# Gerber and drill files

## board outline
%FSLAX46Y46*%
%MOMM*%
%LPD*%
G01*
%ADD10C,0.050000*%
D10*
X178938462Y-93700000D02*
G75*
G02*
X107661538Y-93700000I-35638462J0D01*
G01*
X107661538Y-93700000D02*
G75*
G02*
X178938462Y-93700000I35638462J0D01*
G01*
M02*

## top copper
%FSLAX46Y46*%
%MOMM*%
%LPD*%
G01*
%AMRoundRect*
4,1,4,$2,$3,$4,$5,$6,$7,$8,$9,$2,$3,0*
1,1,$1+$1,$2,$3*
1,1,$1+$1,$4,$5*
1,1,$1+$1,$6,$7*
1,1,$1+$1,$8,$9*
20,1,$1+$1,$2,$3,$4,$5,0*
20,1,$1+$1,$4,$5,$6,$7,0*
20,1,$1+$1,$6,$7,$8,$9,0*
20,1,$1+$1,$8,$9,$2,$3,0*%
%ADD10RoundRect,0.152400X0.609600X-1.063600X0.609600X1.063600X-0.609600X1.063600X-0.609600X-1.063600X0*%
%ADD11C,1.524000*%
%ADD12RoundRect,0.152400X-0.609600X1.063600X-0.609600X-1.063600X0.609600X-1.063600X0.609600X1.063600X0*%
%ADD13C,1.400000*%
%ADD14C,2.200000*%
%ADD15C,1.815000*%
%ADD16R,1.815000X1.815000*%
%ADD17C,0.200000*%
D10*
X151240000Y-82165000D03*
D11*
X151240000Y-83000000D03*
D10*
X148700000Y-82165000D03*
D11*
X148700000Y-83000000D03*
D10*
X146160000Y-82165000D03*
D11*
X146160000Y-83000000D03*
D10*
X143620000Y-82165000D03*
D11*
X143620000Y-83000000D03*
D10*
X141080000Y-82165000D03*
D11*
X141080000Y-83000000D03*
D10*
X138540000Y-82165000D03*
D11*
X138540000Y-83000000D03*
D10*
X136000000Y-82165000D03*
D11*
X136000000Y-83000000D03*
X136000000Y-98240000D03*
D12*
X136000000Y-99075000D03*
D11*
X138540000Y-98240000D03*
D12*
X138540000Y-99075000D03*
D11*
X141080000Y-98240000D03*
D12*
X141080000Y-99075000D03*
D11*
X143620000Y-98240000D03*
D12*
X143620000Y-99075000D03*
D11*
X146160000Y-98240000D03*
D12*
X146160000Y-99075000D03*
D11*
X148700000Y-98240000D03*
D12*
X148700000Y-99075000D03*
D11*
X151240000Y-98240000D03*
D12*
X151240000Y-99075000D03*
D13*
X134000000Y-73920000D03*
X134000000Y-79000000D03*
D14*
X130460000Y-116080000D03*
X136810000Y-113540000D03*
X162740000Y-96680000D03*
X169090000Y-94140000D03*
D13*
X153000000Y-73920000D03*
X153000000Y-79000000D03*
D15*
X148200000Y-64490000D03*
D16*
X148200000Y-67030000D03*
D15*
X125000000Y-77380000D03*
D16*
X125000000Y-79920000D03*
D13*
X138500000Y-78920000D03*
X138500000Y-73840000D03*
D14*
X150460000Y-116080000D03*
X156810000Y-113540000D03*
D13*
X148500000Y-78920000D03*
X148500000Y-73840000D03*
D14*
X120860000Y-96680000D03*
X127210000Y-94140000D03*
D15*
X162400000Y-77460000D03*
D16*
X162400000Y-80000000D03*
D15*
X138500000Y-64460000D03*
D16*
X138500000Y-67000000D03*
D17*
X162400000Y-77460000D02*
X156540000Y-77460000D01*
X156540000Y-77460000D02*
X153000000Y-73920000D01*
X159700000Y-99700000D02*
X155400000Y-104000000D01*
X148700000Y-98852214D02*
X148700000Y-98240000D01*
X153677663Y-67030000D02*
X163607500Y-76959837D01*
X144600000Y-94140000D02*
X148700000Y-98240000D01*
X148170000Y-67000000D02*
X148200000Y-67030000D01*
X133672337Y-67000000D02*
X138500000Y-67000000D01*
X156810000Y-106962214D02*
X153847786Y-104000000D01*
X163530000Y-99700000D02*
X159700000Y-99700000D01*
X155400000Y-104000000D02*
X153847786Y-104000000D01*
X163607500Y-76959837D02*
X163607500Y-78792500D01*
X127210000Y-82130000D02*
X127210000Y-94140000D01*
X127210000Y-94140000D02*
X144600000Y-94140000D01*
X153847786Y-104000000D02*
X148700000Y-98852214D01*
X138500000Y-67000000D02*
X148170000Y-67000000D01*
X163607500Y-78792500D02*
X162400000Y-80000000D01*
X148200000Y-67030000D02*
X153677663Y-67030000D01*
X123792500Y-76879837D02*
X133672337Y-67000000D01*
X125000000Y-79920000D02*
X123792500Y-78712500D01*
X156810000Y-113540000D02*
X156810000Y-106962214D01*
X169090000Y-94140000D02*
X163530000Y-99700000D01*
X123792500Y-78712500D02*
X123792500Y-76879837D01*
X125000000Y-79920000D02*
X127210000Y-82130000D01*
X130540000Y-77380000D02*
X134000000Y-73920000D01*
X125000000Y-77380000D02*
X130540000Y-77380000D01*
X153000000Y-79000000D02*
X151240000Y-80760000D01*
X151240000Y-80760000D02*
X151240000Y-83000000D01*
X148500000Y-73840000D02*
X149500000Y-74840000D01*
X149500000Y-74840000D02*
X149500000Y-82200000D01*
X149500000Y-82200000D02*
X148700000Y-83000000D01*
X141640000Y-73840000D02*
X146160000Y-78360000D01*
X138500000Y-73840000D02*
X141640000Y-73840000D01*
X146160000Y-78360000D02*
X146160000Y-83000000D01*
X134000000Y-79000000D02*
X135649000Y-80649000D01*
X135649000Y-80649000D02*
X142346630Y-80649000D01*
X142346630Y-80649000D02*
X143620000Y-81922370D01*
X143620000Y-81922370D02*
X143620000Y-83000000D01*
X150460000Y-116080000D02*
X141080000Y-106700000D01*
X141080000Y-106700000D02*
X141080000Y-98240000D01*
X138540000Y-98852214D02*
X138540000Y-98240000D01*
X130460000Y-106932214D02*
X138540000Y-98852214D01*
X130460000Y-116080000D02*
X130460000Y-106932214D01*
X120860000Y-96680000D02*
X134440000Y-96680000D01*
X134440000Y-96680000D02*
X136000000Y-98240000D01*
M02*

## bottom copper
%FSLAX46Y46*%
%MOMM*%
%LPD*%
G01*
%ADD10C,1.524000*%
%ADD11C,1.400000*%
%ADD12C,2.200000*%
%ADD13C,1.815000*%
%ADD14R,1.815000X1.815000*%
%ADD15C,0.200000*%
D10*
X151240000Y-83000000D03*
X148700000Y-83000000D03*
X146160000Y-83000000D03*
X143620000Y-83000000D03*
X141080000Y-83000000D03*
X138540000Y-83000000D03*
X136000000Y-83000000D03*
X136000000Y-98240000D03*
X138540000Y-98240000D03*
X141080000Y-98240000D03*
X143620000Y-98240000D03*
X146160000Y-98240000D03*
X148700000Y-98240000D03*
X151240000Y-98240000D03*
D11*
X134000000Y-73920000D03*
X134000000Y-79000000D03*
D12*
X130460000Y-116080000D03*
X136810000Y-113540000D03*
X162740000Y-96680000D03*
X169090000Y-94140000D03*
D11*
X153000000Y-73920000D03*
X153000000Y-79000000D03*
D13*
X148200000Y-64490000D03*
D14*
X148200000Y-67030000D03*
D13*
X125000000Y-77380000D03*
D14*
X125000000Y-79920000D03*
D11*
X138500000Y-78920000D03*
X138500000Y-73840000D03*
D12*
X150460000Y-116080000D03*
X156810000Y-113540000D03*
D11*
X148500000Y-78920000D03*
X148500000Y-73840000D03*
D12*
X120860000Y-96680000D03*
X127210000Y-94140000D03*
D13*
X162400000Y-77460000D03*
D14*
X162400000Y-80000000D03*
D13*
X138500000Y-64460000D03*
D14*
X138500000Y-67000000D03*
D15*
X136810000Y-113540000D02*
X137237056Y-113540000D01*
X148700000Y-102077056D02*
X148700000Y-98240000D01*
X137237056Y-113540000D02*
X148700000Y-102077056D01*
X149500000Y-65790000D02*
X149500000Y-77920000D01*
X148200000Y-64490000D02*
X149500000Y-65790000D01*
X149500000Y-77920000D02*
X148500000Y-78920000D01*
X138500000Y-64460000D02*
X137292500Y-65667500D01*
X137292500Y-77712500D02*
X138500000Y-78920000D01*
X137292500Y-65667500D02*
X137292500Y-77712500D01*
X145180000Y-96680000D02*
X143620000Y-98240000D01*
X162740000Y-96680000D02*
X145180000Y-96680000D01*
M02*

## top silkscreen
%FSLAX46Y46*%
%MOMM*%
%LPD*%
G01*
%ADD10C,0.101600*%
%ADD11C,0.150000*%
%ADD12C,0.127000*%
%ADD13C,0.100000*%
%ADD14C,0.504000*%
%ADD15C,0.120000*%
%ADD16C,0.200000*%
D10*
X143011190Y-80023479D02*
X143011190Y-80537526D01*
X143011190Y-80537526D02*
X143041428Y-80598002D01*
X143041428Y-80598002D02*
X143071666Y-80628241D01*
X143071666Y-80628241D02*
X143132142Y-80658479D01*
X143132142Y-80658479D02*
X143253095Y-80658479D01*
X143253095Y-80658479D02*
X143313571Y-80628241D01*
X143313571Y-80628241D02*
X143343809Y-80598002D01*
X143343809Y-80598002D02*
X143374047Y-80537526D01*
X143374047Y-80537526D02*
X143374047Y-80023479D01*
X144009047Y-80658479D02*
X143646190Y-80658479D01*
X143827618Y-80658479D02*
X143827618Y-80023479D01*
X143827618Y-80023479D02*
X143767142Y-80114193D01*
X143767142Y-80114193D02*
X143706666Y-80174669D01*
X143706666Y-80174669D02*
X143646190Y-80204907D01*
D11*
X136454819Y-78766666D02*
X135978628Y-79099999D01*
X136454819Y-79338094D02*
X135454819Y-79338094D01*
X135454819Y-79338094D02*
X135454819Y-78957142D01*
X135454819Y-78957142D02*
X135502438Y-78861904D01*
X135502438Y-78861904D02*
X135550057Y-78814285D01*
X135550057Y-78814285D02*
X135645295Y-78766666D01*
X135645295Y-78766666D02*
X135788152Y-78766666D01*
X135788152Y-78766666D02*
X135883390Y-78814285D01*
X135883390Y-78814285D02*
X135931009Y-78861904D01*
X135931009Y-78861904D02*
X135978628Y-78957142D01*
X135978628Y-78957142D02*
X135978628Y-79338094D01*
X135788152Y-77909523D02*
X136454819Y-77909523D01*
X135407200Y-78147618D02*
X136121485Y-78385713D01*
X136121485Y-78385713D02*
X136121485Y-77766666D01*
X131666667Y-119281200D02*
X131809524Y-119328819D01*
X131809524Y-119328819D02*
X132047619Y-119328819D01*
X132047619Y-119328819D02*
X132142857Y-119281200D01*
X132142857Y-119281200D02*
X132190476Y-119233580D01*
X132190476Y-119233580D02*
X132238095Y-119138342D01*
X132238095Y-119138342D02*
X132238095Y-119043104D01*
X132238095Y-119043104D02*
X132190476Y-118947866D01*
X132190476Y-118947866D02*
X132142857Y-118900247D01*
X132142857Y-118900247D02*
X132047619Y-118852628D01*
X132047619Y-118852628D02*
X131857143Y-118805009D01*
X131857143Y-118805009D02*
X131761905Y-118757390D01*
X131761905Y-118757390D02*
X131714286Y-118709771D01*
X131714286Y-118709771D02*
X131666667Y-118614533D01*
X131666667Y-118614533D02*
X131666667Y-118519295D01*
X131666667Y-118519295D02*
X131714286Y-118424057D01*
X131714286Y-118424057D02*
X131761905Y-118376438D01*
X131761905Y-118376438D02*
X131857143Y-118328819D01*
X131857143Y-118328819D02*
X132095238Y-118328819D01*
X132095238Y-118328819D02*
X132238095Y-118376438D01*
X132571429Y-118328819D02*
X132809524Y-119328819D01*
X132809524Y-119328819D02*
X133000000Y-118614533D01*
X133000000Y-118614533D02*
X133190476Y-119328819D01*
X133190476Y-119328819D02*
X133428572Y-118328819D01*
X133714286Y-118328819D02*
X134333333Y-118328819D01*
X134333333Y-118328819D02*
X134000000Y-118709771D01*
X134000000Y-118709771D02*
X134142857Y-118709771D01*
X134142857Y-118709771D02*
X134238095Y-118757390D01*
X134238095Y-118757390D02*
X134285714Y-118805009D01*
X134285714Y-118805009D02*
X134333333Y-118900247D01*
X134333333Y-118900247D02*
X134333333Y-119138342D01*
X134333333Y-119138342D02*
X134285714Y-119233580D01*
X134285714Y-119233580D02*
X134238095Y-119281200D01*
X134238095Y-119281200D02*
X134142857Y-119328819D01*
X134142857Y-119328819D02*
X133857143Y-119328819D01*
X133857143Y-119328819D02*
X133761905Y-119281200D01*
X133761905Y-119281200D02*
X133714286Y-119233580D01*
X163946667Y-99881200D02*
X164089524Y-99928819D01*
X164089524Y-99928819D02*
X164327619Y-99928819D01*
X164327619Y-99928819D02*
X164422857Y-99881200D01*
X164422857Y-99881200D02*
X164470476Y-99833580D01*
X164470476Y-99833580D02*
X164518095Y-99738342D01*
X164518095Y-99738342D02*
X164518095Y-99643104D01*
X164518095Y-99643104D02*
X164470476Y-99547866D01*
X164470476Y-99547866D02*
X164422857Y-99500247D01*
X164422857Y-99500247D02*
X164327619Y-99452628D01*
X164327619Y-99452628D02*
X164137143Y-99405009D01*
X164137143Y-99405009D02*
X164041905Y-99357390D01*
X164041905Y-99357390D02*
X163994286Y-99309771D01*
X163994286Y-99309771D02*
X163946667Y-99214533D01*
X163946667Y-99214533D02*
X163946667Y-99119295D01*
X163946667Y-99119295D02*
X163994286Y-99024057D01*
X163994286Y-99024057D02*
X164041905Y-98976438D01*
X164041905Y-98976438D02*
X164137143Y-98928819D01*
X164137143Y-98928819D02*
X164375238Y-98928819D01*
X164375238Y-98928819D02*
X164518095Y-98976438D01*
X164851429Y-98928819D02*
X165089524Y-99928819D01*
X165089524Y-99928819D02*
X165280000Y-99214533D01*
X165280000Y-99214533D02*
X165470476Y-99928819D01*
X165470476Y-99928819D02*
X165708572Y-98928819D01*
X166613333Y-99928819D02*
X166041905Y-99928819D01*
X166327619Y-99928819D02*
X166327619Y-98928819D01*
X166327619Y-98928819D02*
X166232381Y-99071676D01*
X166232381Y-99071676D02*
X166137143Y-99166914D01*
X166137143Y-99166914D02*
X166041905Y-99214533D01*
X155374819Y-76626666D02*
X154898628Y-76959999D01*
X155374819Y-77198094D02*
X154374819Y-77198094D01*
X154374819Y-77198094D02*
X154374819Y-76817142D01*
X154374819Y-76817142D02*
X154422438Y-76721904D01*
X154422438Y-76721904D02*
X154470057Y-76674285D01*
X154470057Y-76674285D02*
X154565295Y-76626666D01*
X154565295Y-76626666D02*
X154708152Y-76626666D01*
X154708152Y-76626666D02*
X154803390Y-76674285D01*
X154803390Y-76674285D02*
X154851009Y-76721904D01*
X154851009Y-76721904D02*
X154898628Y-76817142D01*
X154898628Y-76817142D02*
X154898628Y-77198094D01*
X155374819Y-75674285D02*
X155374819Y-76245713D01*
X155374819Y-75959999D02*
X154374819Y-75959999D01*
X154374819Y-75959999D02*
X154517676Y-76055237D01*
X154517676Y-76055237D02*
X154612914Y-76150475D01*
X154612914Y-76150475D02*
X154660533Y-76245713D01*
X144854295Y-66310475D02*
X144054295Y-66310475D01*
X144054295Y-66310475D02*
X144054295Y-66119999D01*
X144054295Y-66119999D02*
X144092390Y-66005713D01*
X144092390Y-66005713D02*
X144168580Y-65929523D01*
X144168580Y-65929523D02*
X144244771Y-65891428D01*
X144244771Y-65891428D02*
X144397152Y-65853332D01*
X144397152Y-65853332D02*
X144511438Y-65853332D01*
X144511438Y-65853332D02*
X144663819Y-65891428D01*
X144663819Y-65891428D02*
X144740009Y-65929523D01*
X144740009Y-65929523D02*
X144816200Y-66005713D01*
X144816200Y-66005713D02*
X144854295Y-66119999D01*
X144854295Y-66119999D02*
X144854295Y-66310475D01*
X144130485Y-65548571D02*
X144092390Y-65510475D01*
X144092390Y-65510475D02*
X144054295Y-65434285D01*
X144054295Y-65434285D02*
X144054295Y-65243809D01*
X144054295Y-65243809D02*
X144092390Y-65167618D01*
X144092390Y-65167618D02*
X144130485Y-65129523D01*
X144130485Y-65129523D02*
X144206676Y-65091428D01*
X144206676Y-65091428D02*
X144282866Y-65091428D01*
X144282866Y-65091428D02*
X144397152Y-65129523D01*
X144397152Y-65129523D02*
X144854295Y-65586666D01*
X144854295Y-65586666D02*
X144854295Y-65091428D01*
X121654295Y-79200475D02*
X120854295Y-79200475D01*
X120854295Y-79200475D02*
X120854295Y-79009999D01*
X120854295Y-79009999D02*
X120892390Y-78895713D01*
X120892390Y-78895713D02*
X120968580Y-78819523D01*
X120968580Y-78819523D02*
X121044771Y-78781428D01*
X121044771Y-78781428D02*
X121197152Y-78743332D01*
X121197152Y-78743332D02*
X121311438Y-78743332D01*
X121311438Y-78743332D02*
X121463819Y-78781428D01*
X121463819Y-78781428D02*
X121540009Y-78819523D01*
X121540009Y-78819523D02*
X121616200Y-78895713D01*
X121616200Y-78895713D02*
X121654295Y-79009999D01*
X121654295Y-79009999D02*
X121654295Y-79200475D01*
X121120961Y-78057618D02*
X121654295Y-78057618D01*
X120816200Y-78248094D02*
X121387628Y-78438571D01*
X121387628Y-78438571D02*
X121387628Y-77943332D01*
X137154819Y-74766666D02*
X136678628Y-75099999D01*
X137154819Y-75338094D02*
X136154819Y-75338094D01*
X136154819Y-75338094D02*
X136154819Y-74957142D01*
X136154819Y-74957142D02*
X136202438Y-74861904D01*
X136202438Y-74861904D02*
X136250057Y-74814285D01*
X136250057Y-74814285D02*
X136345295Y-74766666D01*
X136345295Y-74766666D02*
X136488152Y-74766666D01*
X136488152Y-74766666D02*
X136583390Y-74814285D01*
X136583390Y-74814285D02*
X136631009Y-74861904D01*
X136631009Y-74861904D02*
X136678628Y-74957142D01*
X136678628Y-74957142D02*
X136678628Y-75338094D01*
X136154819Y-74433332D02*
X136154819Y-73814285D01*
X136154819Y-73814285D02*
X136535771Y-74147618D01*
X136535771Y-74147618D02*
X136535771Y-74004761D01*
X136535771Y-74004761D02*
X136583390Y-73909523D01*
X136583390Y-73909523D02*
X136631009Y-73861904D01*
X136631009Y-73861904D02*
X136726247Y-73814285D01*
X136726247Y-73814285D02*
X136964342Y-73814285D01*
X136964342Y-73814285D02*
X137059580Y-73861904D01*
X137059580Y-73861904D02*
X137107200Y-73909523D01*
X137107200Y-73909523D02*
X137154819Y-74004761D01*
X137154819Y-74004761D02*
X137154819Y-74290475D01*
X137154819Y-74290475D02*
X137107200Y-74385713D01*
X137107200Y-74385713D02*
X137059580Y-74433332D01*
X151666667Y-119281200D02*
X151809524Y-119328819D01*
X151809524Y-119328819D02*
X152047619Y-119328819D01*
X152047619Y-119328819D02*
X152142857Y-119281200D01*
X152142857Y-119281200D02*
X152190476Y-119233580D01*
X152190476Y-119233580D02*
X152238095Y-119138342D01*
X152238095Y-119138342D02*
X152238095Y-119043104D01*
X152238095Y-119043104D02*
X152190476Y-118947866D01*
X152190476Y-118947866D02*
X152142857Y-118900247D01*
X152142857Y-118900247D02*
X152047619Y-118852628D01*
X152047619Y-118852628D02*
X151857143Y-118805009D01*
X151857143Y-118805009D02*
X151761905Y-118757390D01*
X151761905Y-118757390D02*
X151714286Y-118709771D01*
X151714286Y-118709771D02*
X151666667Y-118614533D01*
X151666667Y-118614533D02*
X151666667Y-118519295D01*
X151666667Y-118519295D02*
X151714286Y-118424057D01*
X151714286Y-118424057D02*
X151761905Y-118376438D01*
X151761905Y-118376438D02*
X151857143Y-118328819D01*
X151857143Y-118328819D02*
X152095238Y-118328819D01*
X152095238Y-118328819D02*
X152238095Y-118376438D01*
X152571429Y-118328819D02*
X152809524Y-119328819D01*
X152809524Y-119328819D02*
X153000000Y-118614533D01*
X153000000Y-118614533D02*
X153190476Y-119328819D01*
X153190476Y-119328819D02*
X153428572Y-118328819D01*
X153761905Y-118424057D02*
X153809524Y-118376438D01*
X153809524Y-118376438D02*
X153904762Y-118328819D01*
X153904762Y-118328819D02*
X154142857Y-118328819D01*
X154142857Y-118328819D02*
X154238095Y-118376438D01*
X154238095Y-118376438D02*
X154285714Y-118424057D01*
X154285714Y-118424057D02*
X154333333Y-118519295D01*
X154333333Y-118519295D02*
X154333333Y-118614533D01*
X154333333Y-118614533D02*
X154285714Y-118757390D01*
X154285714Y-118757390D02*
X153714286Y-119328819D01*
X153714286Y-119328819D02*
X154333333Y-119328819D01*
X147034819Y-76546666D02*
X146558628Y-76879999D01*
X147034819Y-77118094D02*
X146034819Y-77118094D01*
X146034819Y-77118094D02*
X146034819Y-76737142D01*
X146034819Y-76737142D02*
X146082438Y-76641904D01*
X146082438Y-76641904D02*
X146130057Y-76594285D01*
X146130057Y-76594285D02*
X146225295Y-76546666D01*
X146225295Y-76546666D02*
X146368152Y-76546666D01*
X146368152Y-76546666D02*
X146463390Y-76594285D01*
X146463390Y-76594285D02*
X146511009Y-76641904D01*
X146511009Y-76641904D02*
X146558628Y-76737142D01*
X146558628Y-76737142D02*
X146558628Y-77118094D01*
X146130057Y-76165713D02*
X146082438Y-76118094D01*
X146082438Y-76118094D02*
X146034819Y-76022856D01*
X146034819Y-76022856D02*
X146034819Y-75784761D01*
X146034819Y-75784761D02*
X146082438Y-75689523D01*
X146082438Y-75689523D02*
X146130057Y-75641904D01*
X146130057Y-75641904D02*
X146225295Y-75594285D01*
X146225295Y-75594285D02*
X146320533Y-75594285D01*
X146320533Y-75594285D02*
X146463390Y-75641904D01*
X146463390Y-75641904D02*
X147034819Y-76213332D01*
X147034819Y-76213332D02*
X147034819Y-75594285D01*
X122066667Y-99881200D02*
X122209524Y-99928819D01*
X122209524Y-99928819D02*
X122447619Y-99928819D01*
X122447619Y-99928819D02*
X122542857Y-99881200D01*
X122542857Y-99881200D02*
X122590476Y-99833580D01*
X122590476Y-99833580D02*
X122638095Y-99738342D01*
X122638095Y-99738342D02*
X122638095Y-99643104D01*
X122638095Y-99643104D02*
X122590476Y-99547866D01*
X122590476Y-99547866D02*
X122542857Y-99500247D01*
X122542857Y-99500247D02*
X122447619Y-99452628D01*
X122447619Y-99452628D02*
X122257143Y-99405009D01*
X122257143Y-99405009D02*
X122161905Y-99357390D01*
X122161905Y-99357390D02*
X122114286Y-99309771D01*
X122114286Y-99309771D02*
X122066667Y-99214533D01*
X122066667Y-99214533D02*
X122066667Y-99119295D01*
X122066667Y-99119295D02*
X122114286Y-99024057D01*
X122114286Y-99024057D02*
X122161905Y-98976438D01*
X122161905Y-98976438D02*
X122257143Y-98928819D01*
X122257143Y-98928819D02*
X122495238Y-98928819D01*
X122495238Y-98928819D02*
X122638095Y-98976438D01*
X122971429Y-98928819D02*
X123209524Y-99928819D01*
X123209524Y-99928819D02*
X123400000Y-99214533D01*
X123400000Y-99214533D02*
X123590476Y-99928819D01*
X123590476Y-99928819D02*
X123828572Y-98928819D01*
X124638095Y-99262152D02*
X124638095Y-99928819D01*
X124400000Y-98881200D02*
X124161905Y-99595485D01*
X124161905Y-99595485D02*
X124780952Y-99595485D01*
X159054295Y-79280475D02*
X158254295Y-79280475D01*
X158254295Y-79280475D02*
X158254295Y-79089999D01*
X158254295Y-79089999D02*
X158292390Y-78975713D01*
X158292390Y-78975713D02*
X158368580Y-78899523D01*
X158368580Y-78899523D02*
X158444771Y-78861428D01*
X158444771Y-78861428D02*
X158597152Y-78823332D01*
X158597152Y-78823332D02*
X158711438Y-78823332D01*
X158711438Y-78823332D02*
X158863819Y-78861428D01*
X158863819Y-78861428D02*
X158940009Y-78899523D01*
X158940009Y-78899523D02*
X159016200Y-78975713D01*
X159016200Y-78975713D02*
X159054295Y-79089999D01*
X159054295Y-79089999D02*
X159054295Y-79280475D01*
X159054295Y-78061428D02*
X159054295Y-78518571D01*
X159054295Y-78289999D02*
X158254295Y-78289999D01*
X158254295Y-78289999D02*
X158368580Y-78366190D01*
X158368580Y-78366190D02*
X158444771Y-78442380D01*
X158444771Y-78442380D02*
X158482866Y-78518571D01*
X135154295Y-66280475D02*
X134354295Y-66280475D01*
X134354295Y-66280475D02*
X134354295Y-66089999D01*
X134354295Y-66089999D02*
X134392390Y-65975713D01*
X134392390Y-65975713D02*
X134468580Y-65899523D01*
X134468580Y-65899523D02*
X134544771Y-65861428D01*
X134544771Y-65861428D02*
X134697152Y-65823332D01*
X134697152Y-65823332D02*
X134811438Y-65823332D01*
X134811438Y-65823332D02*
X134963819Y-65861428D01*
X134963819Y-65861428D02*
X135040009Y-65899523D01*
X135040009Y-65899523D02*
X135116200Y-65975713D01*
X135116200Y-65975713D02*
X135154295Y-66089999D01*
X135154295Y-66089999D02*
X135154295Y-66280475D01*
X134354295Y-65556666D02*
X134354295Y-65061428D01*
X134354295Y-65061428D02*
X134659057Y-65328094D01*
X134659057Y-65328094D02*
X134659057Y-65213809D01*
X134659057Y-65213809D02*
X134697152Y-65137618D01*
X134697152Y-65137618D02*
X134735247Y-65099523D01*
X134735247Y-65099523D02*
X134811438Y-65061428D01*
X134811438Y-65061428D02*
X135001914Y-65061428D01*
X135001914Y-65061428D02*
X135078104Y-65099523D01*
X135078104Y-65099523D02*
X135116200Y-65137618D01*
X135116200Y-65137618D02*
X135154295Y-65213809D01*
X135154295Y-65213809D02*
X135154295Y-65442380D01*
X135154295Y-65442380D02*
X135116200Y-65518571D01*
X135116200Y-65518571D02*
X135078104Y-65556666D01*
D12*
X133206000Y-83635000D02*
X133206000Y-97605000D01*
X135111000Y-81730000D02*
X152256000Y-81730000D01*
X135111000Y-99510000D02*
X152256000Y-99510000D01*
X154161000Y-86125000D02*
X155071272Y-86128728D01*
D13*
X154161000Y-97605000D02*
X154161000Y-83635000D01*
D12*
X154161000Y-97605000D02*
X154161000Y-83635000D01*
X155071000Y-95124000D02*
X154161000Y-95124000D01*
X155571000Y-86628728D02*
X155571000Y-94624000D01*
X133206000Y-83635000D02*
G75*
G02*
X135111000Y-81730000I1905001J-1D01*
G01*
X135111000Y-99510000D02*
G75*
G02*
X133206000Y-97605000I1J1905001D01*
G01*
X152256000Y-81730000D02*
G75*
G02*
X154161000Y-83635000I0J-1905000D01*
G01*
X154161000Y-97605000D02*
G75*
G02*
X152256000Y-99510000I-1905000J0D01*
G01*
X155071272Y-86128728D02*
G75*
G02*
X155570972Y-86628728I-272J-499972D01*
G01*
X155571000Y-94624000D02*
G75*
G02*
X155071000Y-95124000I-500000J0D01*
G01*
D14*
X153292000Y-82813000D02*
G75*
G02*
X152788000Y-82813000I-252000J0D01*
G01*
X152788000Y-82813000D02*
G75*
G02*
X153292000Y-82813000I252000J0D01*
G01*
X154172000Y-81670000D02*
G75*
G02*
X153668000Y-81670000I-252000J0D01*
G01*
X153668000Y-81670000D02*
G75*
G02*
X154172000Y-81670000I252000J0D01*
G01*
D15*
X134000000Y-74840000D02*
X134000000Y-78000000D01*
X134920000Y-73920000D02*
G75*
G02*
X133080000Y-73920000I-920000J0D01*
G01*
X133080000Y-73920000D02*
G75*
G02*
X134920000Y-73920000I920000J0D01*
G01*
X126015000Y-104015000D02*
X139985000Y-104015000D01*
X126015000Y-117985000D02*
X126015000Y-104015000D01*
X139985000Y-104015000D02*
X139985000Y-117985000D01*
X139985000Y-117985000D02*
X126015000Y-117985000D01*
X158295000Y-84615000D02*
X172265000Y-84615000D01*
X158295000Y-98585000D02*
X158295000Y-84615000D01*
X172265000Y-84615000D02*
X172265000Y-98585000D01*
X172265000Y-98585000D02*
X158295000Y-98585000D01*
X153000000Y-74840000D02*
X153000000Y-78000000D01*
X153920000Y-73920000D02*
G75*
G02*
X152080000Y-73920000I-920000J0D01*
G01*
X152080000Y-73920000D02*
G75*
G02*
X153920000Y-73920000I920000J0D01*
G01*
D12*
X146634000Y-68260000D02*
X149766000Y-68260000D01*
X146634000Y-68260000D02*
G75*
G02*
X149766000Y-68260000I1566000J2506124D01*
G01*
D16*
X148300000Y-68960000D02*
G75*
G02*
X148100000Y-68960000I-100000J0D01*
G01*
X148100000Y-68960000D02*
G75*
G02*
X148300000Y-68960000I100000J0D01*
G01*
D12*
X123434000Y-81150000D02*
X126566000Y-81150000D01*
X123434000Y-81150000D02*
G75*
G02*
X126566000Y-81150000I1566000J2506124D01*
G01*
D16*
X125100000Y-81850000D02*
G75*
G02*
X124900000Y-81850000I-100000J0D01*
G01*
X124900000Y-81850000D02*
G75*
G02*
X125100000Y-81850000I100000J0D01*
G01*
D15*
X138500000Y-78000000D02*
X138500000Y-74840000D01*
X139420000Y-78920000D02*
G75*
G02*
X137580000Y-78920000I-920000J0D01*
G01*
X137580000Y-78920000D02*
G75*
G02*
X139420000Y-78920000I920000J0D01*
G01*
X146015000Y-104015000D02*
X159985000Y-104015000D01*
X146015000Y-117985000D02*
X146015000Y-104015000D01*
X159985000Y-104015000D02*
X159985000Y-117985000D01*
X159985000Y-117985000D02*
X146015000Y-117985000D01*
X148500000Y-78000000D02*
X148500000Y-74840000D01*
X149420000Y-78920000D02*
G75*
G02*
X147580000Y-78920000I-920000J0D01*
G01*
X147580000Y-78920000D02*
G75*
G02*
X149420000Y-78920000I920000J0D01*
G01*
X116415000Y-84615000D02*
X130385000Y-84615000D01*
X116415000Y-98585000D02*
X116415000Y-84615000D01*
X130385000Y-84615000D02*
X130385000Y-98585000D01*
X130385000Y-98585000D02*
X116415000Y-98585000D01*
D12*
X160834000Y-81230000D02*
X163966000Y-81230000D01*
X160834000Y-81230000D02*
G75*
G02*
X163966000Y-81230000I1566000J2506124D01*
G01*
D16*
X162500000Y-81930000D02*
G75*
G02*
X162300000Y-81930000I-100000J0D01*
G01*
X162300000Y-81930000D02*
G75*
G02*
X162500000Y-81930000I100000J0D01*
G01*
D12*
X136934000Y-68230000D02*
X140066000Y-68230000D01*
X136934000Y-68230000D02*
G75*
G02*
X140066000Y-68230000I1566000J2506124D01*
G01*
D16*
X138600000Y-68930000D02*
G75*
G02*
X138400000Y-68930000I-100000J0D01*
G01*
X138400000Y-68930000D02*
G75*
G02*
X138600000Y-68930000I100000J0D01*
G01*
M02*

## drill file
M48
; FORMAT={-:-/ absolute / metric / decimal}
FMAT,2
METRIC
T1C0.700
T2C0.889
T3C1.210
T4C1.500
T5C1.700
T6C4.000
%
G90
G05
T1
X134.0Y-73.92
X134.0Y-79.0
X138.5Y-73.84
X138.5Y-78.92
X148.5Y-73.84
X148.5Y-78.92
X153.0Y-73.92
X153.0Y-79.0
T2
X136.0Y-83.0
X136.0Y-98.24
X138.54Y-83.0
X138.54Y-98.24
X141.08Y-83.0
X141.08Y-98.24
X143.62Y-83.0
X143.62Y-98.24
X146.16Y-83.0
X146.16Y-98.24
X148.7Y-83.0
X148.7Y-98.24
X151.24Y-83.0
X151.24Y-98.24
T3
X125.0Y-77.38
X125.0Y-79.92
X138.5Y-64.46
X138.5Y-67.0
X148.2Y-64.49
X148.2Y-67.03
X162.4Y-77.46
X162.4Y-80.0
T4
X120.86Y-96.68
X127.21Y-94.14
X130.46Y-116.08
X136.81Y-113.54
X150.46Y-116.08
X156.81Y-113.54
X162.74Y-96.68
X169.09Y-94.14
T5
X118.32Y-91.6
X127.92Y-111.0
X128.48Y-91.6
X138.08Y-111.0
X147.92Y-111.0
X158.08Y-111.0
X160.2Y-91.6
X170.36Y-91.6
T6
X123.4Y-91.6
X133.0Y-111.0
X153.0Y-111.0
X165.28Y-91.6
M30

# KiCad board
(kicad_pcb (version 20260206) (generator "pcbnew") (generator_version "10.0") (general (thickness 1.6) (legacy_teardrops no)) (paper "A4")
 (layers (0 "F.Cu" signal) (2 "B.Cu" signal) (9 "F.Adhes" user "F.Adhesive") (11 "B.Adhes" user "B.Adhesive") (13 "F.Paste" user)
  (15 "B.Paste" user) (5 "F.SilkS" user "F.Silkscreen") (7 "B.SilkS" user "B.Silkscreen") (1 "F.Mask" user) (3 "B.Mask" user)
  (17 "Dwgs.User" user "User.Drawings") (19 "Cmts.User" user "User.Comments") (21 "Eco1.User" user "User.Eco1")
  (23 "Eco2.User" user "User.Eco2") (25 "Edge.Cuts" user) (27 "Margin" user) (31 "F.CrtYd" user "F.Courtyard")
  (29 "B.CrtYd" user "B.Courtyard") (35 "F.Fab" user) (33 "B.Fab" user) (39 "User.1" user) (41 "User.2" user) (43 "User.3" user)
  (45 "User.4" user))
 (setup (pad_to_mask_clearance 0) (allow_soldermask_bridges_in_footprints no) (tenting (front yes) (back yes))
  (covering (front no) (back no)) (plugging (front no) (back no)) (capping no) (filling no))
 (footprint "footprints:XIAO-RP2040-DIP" (layer "F.Cu") (at 143.62 90.62)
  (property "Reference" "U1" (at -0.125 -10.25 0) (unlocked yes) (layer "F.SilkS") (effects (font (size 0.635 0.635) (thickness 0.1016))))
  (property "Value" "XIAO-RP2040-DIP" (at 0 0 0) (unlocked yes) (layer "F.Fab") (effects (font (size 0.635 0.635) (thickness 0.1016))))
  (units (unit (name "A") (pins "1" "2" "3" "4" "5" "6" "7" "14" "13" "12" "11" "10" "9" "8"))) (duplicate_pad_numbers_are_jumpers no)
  (fp_line (start -10.414 -6.985) (end -10.414 6.985) (stroke (width 0.127) (type solid)) (layer "F.SilkS"))
  (fp_line (start -8.509 -8.89) (end 8.636 -8.89) (stroke (width 0.127) (type solid)) (layer "F.SilkS"))
  (fp_line (start -8.509 8.89) (end 8.636 8.89) (stroke (width 0.127) (type solid)) (layer "F.SilkS"))
  (fp_line (start 10.541 -4.495) (end 11.451272 -4.491272) (stroke (width 0.127) (type solid)) (layer "F.SilkS"))
  (fp_line (start 10.541 6.985) (end 10.541 -6.985) (stroke (width 0.1) (type solid)) (layer "F.SilkS"))
  (fp_line (start 10.541 6.985) (end 10.541 -6.985) (stroke (width 0.127) (type solid)) (layer "F.SilkS"))
  (fp_line (start 11.451 4.504) (end 10.541 4.504) (stroke (width 0.127) (type solid)) (layer "F.SilkS"))
  (fp_line (start 11.951 -3.991272) (end 11.951 4.004) (stroke (width 0.127) (type solid)) (layer "F.SilkS"))
  (fp_arc (start -10.414 -6.985) (mid -9.856038 -8.332038) (end -8.509 -8.89) (stroke (width 0.127) (type solid)) (layer "F.SilkS"))
  (fp_arc (start -8.509 8.89) (mid -9.856038 8.332038) (end -10.414 6.985) (stroke (width 0.127) (type solid)) (layer "F.SilkS"))
  (fp_arc (start 8.636 -8.89) (mid 9.983038 -8.332038) (end 10.541 -6.985) (stroke (width 0.127) (type solid)) (layer "F.SilkS"))
  (fp_arc (start 10.541 6.985) (mid 9.983038 8.332038) (end 8.636 8.89) (stroke (width 0.127) (type solid)) (layer "F.SilkS"))
  (fp_arc (start 11.451272 -4.491272) (mid 11.804644 -4.344724) (end 11.951 -3.991272) (stroke (width 0.127) (type default))
   (layer "F.SilkS"))
  (fp_arc (start 11.951 4.004) (mid 11.804553 4.357553) (end 11.451 4.504) (stroke (width 0.127) (type default)) (layer "F.SilkS"))
  (fp_circle (center 9.42 -7.807) (end 9.674 -7.807) (stroke (width 0.5) (type solid)) (fill yes) (layer "F.SilkS"))
  (fp_circle (center 10.3 -8.95) (end 10.554 -8.95) (stroke (width 0.5) (type solid)) (fill yes) (layer "F.SilkS"))
  (pad "1" smd roundrect (at 7.62 -8.455 90) (size 2.432 1.524) (layers "F.Cu" "F.Mask") (roundrect_rratio 0.1) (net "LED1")
   (thermal_bridge_angle 45))
  (pad "1" thru_hole circle (at 7.62 -7.62 90) (size 1.524 1.524) (drill 0.889) (layers "*.Cu" "*.Mask") (remove_unused_layers no)
   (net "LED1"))
  (pad "2" smd roundrect (at 5.08 -8.455 90) (size 2.432 1.524) (layers "F.Cu" "F.Mask") (roundrect_rratio 0.1) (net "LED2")
   (thermal_bridge_angle 45))
  (pad "2" thru_hole circle (at 5.08 -7.62 90) (size 1.524 1.524) (drill 0.889) (layers "*.Cu" "*.Mask") (remove_unused_layers no)
   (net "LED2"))
  (pad "3" smd roundrect (at 2.54 -8.455 90) (size 2.432 1.524) (layers "F.Cu" "F.Mask") (roundrect_rratio 0.1) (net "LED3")
   (thermal_bridge_angle 45))
  (pad "3" thru_hole circle (at 2.54 -7.62 90) (size 1.524 1.524) (drill 0.889) (layers "*.Cu" "*.Mask") (remove_unused_layers no)
   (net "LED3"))
  (pad "4" smd roundrect (at 0 -8.455 90) (size 2.432 1.524) (layers "F.Cu" "F.Mask") (roundrect_rratio 0.1) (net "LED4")
   (thermal_bridge_angle 45))
  (pad "4" thru_hole circle (at 0 -7.62 90) (size 1.524 1.524) (drill 0.889) (layers "*.Cu" "*.Mask") (remove_unused_layers no) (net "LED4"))
  (pad "5" smd roundrect (at -2.54 -8.455 90) (size 2.432 1.524) (layers "F.Cu" "F.Mask") (roundrect_rratio 0.1)
   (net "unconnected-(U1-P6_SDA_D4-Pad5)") (thermal_bridge_angle 45))
  (pad "5" thru_hole circle (at -2.54 -7.62 90) (size 1.524 1.524) (drill 0.889) (layers "*.Cu" "*.Mask") (remove_unused_layers no)
   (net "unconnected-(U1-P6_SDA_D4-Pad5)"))
  (pad "6" smd roundrect (at -5.08 -8.455 90) (size 2.432 1.524) (layers "F.Cu" "F.Mask") (roundrect_rratio 0.1)
   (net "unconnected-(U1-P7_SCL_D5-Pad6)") (thermal_bridge_angle 45))
  (pad "6" thru_hole circle (at -5.08 -7.62 90) (size 1.524 1.524) (drill 0.889) (layers "*.Cu" "*.Mask") (remove_unused_layers no)
   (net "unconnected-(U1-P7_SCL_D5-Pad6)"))
  (pad "7" smd roundrect (at -7.62 -8.455 90) (size 2.432 1.524) (layers "F.Cu" "F.Mask") (roundrect_rratio 0.1)
   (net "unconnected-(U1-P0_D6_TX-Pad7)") (thermal_bridge_angle 45))
  (pad "7" thru_hole circle (at -7.62 -7.62 90) (size 1.524 1.524) (drill 0.889) (layers "*.Cu" "*.Mask") (remove_unused_layers no)
   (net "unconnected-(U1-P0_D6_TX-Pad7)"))
  (pad "8" thru_hole circle (at -7.62 7.62 270) (size 1.524 1.524) (drill 0.889) (layers "*.Cu" "*.Mask") (remove_unused_layers no)
   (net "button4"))
  (pad "8" smd roundrect (at -7.62 8.455 270) (size 2.432 1.524) (layers "F.Cu" "F.Mask") (roundrect_rratio 0.1) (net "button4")
   (thermal_bridge_angle 45))
  (pad "9" thru_hole circle (at -5.08 7.62 270) (size 1.524 1.524) (drill 0.889) (layers "*.Cu" "*.Mask") (remove_unused_layers no)
   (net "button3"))
  (pad "9" smd roundrect (at -5.08 8.455 270) (size 2.432 1.524) (layers "F.Cu" "F.Mask") (roundrect_rratio 0.1) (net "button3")
   (thermal_bridge_angle 45))
  (pad "10" thru_hole circle (at -2.54 7.62 270) (size 1.524 1.524) (drill 0.889) (layers "*.Cu" "*.Mask") (remove_unused_layers no)
   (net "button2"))
  (pad "10" smd roundrect (at -2.54 8.455 270) (size 2.432 1.524) (layers "F.Cu" "F.Mask") (roundrect_rratio 0.1) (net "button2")
   (thermal_bridge_angle 45))
  (pad "11" thru_hole circle (at 0 7.62 270) (size 1.524 1.524) (drill 0.889) (layers "*.Cu" "*.Mask") (remove_unused_layers no)
   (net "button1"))
  (pad "11" smd roundrect (at 0 8.455 270) (size 2.432 1.524) (layers "F.Cu" "F.Mask") (roundrect_rratio 0.1) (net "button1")
   (thermal_bridge_angle 45))
  (pad "12" thru_hole circle (at 2.54 7.62 270) (size 1.524 1.524) (drill 0.889) (layers "*.Cu" "*.Mask") (remove_unused_layers no)
   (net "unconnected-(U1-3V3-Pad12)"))
  (pad "12" smd roundrect (at 2.54 8.455 270) (size 2.432 1.524) (layers "F.Cu" "F.Mask") (roundrect_rratio 0.1)
   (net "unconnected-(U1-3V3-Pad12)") (thermal_bridge_angle 45))
  (pad "13" thru_hole circle (at 5.08 7.62 270) (size 1.524 1.524) (drill 0.889) (layers "*.Cu" "*.Mask") (remove_unused_layers no)
   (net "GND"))
  (pad "13" smd roundrect (at 5.08 8.455 270) (size 2.432 1.524) (layers "F.Cu" "F.Mask") (roundrect_rratio 0.1) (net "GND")
   (thermal_bridge_angle 45))
  (pad "14" thru_hole circle (at 7.62 7.62 270) (size 1.524 1.524) (drill 0.889) (layers "*.Cu" "*.Mask") (remove_unused_layers no)
   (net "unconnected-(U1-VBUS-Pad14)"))
  (pad "14" smd roundrect (at 7.62 8.455 270) (size 2.432 1.524) (layers "F.Cu" "F.Mask") (roundrect_rratio 0.1)
   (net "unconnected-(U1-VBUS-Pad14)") (thermal_bridge_angle 45)))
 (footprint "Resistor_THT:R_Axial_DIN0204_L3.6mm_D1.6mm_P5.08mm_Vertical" (layer "F.Cu") (at 134 73.92 -90)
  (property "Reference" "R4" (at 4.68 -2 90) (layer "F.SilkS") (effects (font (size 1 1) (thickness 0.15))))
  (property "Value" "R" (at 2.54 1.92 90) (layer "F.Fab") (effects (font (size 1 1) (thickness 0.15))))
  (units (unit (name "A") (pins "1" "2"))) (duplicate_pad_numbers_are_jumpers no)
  (fp_line (start 0.92 0) (end 4.08 0) (stroke (width 0.12) (type solid)) (layer "F.SilkS"))
  (fp_circle (center 0 0) (end 0.92 0) (stroke (width 0.12) (type solid)) (fill no) (layer "F.SilkS"))
  (pad "1" thru_hole circle (at 0 0 270) (size 1.4 1.4) (drill 0.7) (layers "*.Cu" "*.Mask") (remove_unused_layers no) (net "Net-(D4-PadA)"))
  (pad "2" thru_hole circle (at 5.08 0 270) (size 1.4 1.4) (drill 0.7) (layers "*.Cu" "*.Mask") (remove_unused_layers no) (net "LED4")))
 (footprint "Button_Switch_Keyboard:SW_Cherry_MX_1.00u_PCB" (layer "F.Cu") (at 130.46 116.08 180)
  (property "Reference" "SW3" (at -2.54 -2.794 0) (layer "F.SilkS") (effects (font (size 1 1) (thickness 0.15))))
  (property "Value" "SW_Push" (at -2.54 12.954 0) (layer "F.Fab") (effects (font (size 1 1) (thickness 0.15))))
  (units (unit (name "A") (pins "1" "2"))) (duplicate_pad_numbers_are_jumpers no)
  (fp_line (start 4.445 12.065) (end -9.525 12.065) (stroke (width 0.12) (type solid)) (layer "F.SilkS"))
  (fp_line (start 4.445 -1.905) (end 4.445 12.065) (stroke (width 0.12) (type solid)) (layer "F.SilkS"))
  (fp_line (start -9.525 12.065) (end -9.525 -1.905) (stroke (width 0.12) (type solid)) (layer "F.SilkS"))
  (fp_line (start -9.525 -1.905) (end 4.445 -1.905) (stroke (width 0.12) (type solid)) (layer "F.SilkS"))
  (pad "" np_thru_hole circle (at -7.62 5.08 180) (size 1.7 1.7) (drill 1.7) (layers "*.Cu" "*.Mask"))
  (pad "" np_thru_hole circle (at -2.54 5.08 180) (size 4 4) (drill 4) (layers "*.Cu" "*.Mask"))
  (pad "" np_thru_hole circle (at 2.54 5.08 180) (size 1.7 1.7) (drill 1.7) (layers "*.Cu" "*.Mask"))
  (pad "1" thru_hole circle (at 0 0 180) (size 2.2 2.2) (drill 1.5) (layers "*.Cu" "*.Mask") (remove_unused_layers no) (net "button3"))
  (pad "2" thru_hole circle (at -6.35 2.54 180) (size 2.2 2.2) (drill 1.5) (layers "*.Cu" "*.Mask") (remove_unused_layers no) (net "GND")))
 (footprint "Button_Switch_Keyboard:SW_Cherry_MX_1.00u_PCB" (layer "F.Cu") (at 162.74 96.68 180)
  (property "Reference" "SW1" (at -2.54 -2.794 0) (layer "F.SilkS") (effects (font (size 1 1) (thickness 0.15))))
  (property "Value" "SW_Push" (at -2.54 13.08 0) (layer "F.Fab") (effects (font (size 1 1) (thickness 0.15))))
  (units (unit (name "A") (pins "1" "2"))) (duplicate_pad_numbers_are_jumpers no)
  (fp_line (start 4.445 12.065) (end -9.525 12.065) (stroke (width 0.12) (type solid)) (layer "F.SilkS"))
  (fp_line (start 4.445 -1.905) (end 4.445 12.065) (stroke (width 0.12) (type solid)) (layer "F.SilkS"))
  (fp_line (start -9.525 12.065) (end -9.525 -1.905) (stroke (width 0.12) (type solid)) (layer "F.SilkS"))
  (fp_line (start -9.525 -1.905) (end 4.445 -1.905) (stroke (width 0.12) (type solid)) (layer "F.SilkS"))
  (pad "" np_thru_hole circle (at -7.62 5.08 180) (size 1.7 1.7) (drill 1.7) (layers "*.Cu" "*.Mask"))
  (pad "" np_thru_hole circle (at -2.54 5.08 180) (size 4 4) (drill 4) (layers "*.Cu" "*.Mask"))
  (pad "" np_thru_hole circle (at 2.54 5.08 180) (size 1.7 1.7) (drill 1.7) (layers "*.Cu" "*.Mask"))
  (pad "1" thru_hole circle (at 0 0 180) (size 2.2 2.2) (drill 1.5) (layers "*.Cu" "*.Mask") (remove_unused_layers no) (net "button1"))
  (pad "2" thru_hole circle (at -6.35 2.54 180) (size 2.2 2.2) (drill 1.5) (layers "*.Cu" "*.Mask") (remove_unused_layers no) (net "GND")))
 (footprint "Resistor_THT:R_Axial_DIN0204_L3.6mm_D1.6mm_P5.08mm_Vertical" (layer "F.Cu") (at 153 73.92 -90)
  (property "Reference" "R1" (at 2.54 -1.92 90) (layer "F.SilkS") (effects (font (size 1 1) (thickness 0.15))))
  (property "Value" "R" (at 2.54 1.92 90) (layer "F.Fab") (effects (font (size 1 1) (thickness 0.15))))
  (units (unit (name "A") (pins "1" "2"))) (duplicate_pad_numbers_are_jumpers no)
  (fp_line (start 0.92 0) (end 4.08 0) (stroke (width 0.12) (type solid)) (layer "F.SilkS"))
  (fp_circle (center 0 0) (end 0.92 0) (stroke (width 0.12) (type solid)) (fill no) (layer "F.SilkS"))
  (pad "1" thru_hole circle (at 0 0 270) (size 1.4 1.4) (drill 0.7) (layers "*.Cu" "*.Mask") (remove_unused_layers no) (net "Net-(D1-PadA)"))
  (pad "2" thru_hole circle (at 5.08 0 270) (size 1.4 1.4) (drill 0.7) (layers "*.Cu" "*.Mask") (remove_unused_layers no) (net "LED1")))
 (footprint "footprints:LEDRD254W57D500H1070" (layer "F.Cu") (at 148.2 65.76 90)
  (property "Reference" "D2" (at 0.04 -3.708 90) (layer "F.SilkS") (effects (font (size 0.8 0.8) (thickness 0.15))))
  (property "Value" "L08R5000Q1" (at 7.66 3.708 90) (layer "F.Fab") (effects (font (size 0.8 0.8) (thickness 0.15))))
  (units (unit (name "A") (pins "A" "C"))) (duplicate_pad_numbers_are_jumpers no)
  (fp_line (start -2.5 -1.566) (end -2.5 1.566) (stroke (width 0.127) (type solid)) (layer "F.SilkS"))
  (fp_arc (start -2.5 -1.566) (mid 2.961291 0) (end -2.5 1.566) (stroke (width 0.127) (type solid)) (layer "F.SilkS"))
  (fp_circle (center -3.2 0) (end -3.1 0) (stroke (width 0.2) (type solid)) (fill no) (layer "F.SilkS"))
  (pad "A" thru_hole circle (at 1.27 0 90) (size 1.815 1.815) (drill 1.21) (layers "*.Cu" "*.Mask") (remove_unused_layers no)
   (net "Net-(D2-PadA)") (solder_mask_margin 0.102))
  (pad "C" thru_hole rect (at -1.27 0 90) (size 1.815 1.815) (drill 1.21) (layers "*.Cu" "*.Mask") (remove_unused_layers no) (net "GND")
   (solder_mask_margin 0.102)))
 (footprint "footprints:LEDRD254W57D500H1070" (layer "F.Cu") (at 125 78.65 90)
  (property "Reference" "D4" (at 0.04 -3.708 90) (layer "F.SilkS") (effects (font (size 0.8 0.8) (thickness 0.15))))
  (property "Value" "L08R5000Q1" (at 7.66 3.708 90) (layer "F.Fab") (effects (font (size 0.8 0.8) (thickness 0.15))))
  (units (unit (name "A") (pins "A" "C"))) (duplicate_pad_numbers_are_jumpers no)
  (fp_line (start -2.5 -1.566) (end -2.5 1.566) (stroke (width 0.127) (type solid)) (layer "F.SilkS"))
  (fp_arc (start -2.5 -1.566) (mid 2.961291 0) (end -2.5 1.566) (stroke (width 0.127) (type solid)) (layer "F.SilkS"))
  (fp_circle (center -3.2 0) (end -3.1 0) (stroke (width 0.2) (type solid)) (fill no) (layer "F.SilkS"))
  (pad "A" thru_hole circle (at 1.27 0 90) (size 1.815 1.815) (drill 1.21) (layers "*.Cu" "*.Mask") (remove_unused_layers no)
   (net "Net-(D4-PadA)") (solder_mask_margin 0.102))
  (pad "C" thru_hole rect (at -1.27 0 90) (size 1.815 1.815) (drill 1.21) (layers "*.Cu" "*.Mask") (remove_unused_layers no) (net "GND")
   (solder_mask_margin 0.102)))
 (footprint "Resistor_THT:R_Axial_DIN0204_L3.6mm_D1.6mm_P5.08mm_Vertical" (layer "F.Cu") (at 138.5 78.92 90)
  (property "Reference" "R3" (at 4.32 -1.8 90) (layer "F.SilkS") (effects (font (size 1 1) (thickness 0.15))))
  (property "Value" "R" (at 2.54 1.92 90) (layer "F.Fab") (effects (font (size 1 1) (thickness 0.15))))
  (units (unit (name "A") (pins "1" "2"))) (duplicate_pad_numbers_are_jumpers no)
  (fp_line (start 0.92 0) (end 4.08 0) (stroke (width 0.12) (type solid)) (layer "F.SilkS"))
  (fp_circle (center 0 0) (end 0.92 0) (stroke (width 0.12) (type solid)) (fill no) (layer "F.SilkS"))
  (pad "1" thru_hole circle (at 0 0 90) (size 1.4 1.4) (drill 0.7) (layers "*.Cu" "*.Mask") (remove_unused_layers no) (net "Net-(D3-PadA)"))
  (pad "2" thru_hole circle (at 5.08 0 90) (size 1.4 1.4) (drill 0.7) (layers "*.Cu" "*.Mask") (remove_unused_layers no) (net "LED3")))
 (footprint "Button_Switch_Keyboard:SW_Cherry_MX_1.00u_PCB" (layer "F.Cu") (at 150.46 116.08 180)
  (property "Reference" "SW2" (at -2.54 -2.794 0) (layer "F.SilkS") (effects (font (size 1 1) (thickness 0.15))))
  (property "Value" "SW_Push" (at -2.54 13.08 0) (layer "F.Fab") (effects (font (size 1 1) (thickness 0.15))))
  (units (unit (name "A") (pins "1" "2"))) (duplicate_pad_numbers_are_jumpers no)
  (fp_line (start 4.445 12.065) (end -9.525 12.065) (stroke (width 0.12) (type solid)) (layer "F.SilkS"))
  (fp_line (start 4.445 -1.905) (end 4.445 12.065) (stroke (width 0.12) (type solid)) (layer "F.SilkS"))
  (fp_line (start -9.525 12.065) (end -9.525 -1.905) (stroke (width 0.12) (type solid)) (layer "F.SilkS"))
  (fp_line (start -9.525 -1.905) (end 4.445 -1.905) (stroke (width 0.12) (type solid)) (layer "F.SilkS"))
  (pad "" np_thru_hole circle (at -7.62 5.08 180) (size 1.7 1.7) (drill 1.7) (layers "*.Cu" "*.Mask"))
  (pad "" np_thru_hole circle (at -2.54 5.08 180) (size 4 4) (drill 4) (layers "*.Cu" "*.Mask"))
  (pad "" np_thru_hole circle (at 2.54 5.08 180) (size 1.7 1.7) (drill 1.7) (layers "*.Cu" "*.Mask"))
  (pad "1" thru_hole circle (at 0 0 180) (size 2.2 2.2) (drill 1.5) (layers "*.Cu" "*.Mask") (remove_unused_layers no) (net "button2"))
  (pad "2" thru_hole circle (at -6.35 2.54 180) (size 2.2 2.2) (drill 1.5) (layers "*.Cu" "*.Mask") (remove_unused_layers no) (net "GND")))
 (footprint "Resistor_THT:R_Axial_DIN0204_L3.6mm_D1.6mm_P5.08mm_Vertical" (layer "F.Cu") (at 148.5 78.92 90)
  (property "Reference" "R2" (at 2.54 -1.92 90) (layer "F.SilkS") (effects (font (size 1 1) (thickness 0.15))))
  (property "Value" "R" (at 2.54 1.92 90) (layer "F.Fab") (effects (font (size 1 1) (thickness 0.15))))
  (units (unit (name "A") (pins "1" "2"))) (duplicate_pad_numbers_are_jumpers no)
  (fp_line (start 0.92 0) (end 4.08 0) (stroke (width 0.12) (type solid)) (layer "F.SilkS"))
  (fp_circle (center 0 0) (end 0.92 0) (stroke (width 0.12) (type solid)) (fill no) (layer "F.SilkS"))
  (pad "1" thru_hole circle (at 0 0 90) (size 1.4 1.4) (drill 0.7) (layers "*.Cu" "*.Mask") (remove_unused_layers no) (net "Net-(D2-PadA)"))
  (pad "2" thru_hole circle (at 5.08 0 90) (size 1.4 1.4) (drill 0.7) (layers "*.Cu" "*.Mask") (remove_unused_layers no) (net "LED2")))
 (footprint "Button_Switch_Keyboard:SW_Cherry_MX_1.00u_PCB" (layer "F.Cu") (at 120.86 96.68 180)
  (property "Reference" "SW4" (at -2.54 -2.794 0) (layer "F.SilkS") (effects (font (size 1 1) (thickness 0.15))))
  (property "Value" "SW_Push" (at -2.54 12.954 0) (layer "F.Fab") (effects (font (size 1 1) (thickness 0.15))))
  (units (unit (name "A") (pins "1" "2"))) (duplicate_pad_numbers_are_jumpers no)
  (fp_line (start 4.445 12.065) (end -9.525 12.065) (stroke (width 0.12) (type solid)) (layer "F.SilkS"))
  (fp_line (start 4.445 -1.905) (end 4.445 12.065) (stroke (width 0.12) (type solid)) (layer "F.SilkS"))
  (fp_line (start -9.525 12.065) (end -9.525 -1.905) (stroke (width 0.12) (type solid)) (layer "F.SilkS"))
  (fp_line (start -9.525 -1.905) (end 4.445 -1.905) (stroke (width 0.12) (type solid)) (layer "F.SilkS"))
  (pad "" np_thru_hole circle (at -7.62 5.08 180) (size 1.7 1.7) (drill 1.7) (layers "*.Cu" "*.Mask"))
  (pad "" np_thru_hole circle (at -2.54 5.08 180) (size 4 4) (drill 4) (layers "*.Cu" "*.Mask"))
  (pad "" np_thru_hole circle (at 2.54 5.08 180) (size 1.7 1.7) (drill 1.7) (layers "*.Cu" "*.Mask"))
  (pad "1" thru_hole circle (at 0 0 180) (size 2.2 2.2) (drill 1.5) (layers "*.Cu" "*.Mask") (remove_unused_layers no) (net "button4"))
  (pad "2" thru_hole circle (at -6.35 2.54 180) (size 2.2 2.2) (drill 1.5) (layers "*.Cu" "*.Mask") (remove_unused_layers no) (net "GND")))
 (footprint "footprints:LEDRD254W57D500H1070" (layer "F.Cu") (at 162.4 78.73 90)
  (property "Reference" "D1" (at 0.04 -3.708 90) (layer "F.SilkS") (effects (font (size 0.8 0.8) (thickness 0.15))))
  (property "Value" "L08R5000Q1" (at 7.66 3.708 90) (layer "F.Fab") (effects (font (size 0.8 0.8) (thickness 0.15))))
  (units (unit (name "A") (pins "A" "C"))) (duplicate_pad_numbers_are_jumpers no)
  (fp_line (start -2.5 -1.566) (end -2.5 1.566) (stroke (width 0.127) (type solid)) (layer "F.SilkS"))
  (fp_arc (start -2.5 -1.566) (mid 2.961291 0) (end -2.5 1.566) (stroke (width 0.127) (type solid)) (layer "F.SilkS"))
  (fp_circle (center -3.2 0) (end -3.1 0) (stroke (width 0.2) (type solid)) (fill no) (layer "F.SilkS"))
  (pad "A" thru_hole circle (at 1.27 0 90) (size 1.815 1.815) (drill 1.21) (layers "*.Cu" "*.Mask") (remove_unused_layers no)
   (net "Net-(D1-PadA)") (solder_mask_margin 0.102))
  (pad "C" thru_hole rect (at -1.27 0 90) (size 1.815 1.815) (drill 1.21) (layers "*.Cu" "*.Mask") (remove_unused_layers no) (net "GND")
   (solder_mask_margin 0.102)))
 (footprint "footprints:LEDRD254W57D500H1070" (layer "F.Cu") (at 138.5 65.73 90)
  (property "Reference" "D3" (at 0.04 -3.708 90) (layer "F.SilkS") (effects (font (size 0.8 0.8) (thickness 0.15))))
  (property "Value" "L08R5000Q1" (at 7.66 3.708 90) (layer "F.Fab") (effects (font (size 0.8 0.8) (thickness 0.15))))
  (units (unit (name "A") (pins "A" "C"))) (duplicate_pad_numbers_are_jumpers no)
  (fp_line (start -2.5 -1.566) (end -2.5 1.566) (stroke (width 0.127) (type solid)) (layer "F.SilkS"))
  (fp_arc (start -2.5 -1.566) (mid 2.961291 0) (end -2.5 1.566) (stroke (width 0.127) (type solid)) (layer "F.SilkS"))
  (fp_circle (center -3.2 0) (end -3.1 0) (stroke (width 0.2) (type solid)) (fill no) (layer "F.SilkS"))
  (pad "A" thru_hole circle (at 1.27 0 90) (size 1.815 1.815) (drill 1.21) (layers "*.Cu" "*.Mask") (remove_unused_layers no)
   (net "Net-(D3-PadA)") (solder_mask_margin 0.102))
  (pad "C" thru_hole rect (at -1.27 0 90) (size 1.815 1.815) (drill 1.21) (layers "*.Cu" "*.Mask") (remove_unused_layers no) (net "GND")
   (solder_mask_margin 0.102)))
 (gr_circle (center 143.3 93.7) (end 168.6 118.8) (stroke (width 0.05) (type default)) (fill no) (layer "Edge.Cuts"))
 (segment (start 162.4 77.46) (end 156.54 77.46) (width 0.2) (layer "F.Cu") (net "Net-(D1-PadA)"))
 (segment (start 156.54 77.46) (end 153 73.92) (width 0.2) (layer "F.Cu") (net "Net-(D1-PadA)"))
 (segment (start 159.7 99.7) (end 155.4 104) (width 0.2) (layer "F.Cu") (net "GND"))
 (segment (start 148.7 98.852214) (end 148.7 98.24) (width 0.2) (layer "F.Cu") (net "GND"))
 (segment (start 153.677663 67.03) (end 163.6075 76.959837) (width 0.2) (layer "F.Cu") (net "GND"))
 (segment (start 144.6 94.14) (end 148.7 98.24) (width 0.2) (layer "F.Cu") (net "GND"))
 (segment (start 148.17 67) (end 148.2 67.03) (width 0.2) (layer "F.Cu") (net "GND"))
 (segment (start 133.672337 67) (end 138.5 67) (width 0.2) (layer "F.Cu") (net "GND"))
 (segment (start 156.81 106.962214) (end 153.847786 104) (width 0.2) (layer "F.Cu") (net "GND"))
 (segment (start 163.53 99.7) (end 159.7 99.7) (width 0.2) (layer "F.Cu") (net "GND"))
 (segment (start 155.4 104) (end 153.847786 104) (width 0.2) (layer "F.Cu") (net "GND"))
 (segment (start 163.6075 76.959837) (end 163.6075 78.7925) (width 0.2) (layer "F.Cu") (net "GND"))
 (segment (start 127.21 82.13) (end 127.21 94.14) (width 0.2) (layer "F.Cu") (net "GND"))
 (segment (start 127.21 94.14) (end 144.6 94.14) (width 0.2) (layer "F.Cu") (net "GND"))
 (segment (start 153.847786 104) (end 148.7 98.852214) (width 0.2) (layer "F.Cu") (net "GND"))
 (segment (start 138.5 67) (end 148.17 67) (width 0.2) (layer "F.Cu") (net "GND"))
 (segment (start 163.6075 78.7925) (end 162.4 80) (width 0.2) (layer "F.Cu") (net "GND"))
 (segment (start 148.2 67.03) (end 153.677663 67.03) (width 0.2) (layer "F.Cu") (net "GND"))
 (segment (start 123.7925 76.879837) (end 133.672337 67) (width 0.2) (layer "F.Cu") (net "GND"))
 (segment (start 125 79.92) (end 123.7925 78.7125) (width 0.2) (layer "F.Cu") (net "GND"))
 (segment (start 156.81 113.54) (end 156.81 106.962214) (width 0.2) (layer "F.Cu") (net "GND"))
 (segment (start 169.09 94.14) (end 163.53 99.7) (width 0.2) (layer "F.Cu") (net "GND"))
 (segment (start 123.7925 78.7125) (end 123.7925 76.879837) (width 0.2) (layer "F.Cu") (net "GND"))
 (segment (start 125 79.92) (end 127.21 82.13) (width 0.2) (layer "F.Cu") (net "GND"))
 (segment (start 136.81 113.54) (end 137.237056 113.54) (width 0.2) (layer "B.Cu") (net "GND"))
 (segment (start 148.7 102.077056) (end 148.7 98.24) (width 0.2) (layer "B.Cu") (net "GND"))
 (segment (start 137.237056 113.54) (end 148.7 102.077056) (width 0.2) (layer "B.Cu") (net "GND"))
 (segment (start 149.5 65.79) (end 149.5 77.92) (width 0.2) (layer "B.Cu") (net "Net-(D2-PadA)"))
 (segment (start 148.2 64.49) (end 149.5 65.79) (width 0.2) (layer "B.Cu") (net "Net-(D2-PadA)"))
 (segment (start 149.5 77.92) (end 148.5 78.92) (width 0.2) (layer "B.Cu") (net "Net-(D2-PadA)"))
 (segment (start 138.5 64.46) (end 137.2925 65.6675) (width 0.2) (layer "B.Cu") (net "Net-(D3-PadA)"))
 (segment (start 137.2925 77.7125) (end 138.5 78.92) (width 0.2) (layer "B.Cu") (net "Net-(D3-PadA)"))
 (segment (start 137.2925 65.6675) (end 137.2925 77.7125) (width 0.2) (layer "B.Cu") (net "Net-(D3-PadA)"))
 (segment (start 130.54 77.38) (end 134 73.92) (width 0.2) (layer "F.Cu") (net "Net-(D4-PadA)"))
 (segment (start 125 77.38) (end 130.54 77.38) (width 0.2) (layer "F.Cu") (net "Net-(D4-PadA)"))
 (segment (start 153 79) (end 151.24 80.76) (width 0.2) (layer "F.Cu") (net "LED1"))
 (segment (start 151.24 80.76) (end 151.24 83) (width 0.2) (layer "F.Cu") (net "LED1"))
 (segment (start 148.5 73.84) (end 149.5 74.84) (width 0.2) (layer "F.Cu") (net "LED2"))
 (segment (start 149.5 74.84) (end 149.5 82.2) (width 0.2) (layer "F.Cu") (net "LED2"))
 (segment (start 149.5 82.2) (end 148.7 83) (width 0.2) (layer "F.Cu") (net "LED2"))
 (segment (start 141.64 73.84) (end 146.16 78.36) (width 0.2) (layer "F.Cu") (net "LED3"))
 (segment (start 138.5 73.84) (end 141.64 73.84) (width 0.2) (layer "F.Cu") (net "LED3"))
 (segment (start 146.16 78.36) (end 146.16 83) (width 0.2) (layer "F.Cu") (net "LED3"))
 (segment (start 134 79) (end 135.649 80.649) (width 0.2) (layer "F.Cu") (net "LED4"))
 (segment (start 135.649 80.649) (end 142.34663 80.649) (width 0.2) (layer "F.Cu") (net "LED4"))
 (segment (start 142.34663 80.649) (end 143.62 81.92237) (width 0.2) (layer "F.Cu") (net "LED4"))
 (segment (start 143.62 81.92237) (end 143.62 83) (width 0.2) (layer "F.Cu") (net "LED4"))
 (segment (start 145.18 96.68) (end 143.62 98.24) (width 0.2) (layer "B.Cu") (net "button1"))
 (segment (start 162.74 96.68) (end 145.18 96.68) (width 0.2) (layer "B.Cu") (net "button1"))
 (segment (start 150.46 116.08) (end 141.08 106.7) (width 0.2) (layer "F.Cu") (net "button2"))
 (segment (start 141.08 106.7) (end 141.08 98.24) (width 0.2) (layer "F.Cu") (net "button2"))
 (segment (start 138.54 98.852214) (end 138.54 98.24) (width 0.2) (layer "F.Cu") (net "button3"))
 (segment (start 130.46 106.932214) (end 138.54 98.852214) (width 0.2) (layer "F.Cu") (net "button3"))
 (segment (start 130.46 116.08) (end 130.46 106.932214) (width 0.2) (layer "F.Cu") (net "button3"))
 (segment (start 120.86 96.68) (end 134.44 96.68) (width 0.2) (layer "F.Cu") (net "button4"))
 (segment (start 134.44 96.68) (end 136 98.24) (width 0.2) (layer "F.Cu") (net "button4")))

